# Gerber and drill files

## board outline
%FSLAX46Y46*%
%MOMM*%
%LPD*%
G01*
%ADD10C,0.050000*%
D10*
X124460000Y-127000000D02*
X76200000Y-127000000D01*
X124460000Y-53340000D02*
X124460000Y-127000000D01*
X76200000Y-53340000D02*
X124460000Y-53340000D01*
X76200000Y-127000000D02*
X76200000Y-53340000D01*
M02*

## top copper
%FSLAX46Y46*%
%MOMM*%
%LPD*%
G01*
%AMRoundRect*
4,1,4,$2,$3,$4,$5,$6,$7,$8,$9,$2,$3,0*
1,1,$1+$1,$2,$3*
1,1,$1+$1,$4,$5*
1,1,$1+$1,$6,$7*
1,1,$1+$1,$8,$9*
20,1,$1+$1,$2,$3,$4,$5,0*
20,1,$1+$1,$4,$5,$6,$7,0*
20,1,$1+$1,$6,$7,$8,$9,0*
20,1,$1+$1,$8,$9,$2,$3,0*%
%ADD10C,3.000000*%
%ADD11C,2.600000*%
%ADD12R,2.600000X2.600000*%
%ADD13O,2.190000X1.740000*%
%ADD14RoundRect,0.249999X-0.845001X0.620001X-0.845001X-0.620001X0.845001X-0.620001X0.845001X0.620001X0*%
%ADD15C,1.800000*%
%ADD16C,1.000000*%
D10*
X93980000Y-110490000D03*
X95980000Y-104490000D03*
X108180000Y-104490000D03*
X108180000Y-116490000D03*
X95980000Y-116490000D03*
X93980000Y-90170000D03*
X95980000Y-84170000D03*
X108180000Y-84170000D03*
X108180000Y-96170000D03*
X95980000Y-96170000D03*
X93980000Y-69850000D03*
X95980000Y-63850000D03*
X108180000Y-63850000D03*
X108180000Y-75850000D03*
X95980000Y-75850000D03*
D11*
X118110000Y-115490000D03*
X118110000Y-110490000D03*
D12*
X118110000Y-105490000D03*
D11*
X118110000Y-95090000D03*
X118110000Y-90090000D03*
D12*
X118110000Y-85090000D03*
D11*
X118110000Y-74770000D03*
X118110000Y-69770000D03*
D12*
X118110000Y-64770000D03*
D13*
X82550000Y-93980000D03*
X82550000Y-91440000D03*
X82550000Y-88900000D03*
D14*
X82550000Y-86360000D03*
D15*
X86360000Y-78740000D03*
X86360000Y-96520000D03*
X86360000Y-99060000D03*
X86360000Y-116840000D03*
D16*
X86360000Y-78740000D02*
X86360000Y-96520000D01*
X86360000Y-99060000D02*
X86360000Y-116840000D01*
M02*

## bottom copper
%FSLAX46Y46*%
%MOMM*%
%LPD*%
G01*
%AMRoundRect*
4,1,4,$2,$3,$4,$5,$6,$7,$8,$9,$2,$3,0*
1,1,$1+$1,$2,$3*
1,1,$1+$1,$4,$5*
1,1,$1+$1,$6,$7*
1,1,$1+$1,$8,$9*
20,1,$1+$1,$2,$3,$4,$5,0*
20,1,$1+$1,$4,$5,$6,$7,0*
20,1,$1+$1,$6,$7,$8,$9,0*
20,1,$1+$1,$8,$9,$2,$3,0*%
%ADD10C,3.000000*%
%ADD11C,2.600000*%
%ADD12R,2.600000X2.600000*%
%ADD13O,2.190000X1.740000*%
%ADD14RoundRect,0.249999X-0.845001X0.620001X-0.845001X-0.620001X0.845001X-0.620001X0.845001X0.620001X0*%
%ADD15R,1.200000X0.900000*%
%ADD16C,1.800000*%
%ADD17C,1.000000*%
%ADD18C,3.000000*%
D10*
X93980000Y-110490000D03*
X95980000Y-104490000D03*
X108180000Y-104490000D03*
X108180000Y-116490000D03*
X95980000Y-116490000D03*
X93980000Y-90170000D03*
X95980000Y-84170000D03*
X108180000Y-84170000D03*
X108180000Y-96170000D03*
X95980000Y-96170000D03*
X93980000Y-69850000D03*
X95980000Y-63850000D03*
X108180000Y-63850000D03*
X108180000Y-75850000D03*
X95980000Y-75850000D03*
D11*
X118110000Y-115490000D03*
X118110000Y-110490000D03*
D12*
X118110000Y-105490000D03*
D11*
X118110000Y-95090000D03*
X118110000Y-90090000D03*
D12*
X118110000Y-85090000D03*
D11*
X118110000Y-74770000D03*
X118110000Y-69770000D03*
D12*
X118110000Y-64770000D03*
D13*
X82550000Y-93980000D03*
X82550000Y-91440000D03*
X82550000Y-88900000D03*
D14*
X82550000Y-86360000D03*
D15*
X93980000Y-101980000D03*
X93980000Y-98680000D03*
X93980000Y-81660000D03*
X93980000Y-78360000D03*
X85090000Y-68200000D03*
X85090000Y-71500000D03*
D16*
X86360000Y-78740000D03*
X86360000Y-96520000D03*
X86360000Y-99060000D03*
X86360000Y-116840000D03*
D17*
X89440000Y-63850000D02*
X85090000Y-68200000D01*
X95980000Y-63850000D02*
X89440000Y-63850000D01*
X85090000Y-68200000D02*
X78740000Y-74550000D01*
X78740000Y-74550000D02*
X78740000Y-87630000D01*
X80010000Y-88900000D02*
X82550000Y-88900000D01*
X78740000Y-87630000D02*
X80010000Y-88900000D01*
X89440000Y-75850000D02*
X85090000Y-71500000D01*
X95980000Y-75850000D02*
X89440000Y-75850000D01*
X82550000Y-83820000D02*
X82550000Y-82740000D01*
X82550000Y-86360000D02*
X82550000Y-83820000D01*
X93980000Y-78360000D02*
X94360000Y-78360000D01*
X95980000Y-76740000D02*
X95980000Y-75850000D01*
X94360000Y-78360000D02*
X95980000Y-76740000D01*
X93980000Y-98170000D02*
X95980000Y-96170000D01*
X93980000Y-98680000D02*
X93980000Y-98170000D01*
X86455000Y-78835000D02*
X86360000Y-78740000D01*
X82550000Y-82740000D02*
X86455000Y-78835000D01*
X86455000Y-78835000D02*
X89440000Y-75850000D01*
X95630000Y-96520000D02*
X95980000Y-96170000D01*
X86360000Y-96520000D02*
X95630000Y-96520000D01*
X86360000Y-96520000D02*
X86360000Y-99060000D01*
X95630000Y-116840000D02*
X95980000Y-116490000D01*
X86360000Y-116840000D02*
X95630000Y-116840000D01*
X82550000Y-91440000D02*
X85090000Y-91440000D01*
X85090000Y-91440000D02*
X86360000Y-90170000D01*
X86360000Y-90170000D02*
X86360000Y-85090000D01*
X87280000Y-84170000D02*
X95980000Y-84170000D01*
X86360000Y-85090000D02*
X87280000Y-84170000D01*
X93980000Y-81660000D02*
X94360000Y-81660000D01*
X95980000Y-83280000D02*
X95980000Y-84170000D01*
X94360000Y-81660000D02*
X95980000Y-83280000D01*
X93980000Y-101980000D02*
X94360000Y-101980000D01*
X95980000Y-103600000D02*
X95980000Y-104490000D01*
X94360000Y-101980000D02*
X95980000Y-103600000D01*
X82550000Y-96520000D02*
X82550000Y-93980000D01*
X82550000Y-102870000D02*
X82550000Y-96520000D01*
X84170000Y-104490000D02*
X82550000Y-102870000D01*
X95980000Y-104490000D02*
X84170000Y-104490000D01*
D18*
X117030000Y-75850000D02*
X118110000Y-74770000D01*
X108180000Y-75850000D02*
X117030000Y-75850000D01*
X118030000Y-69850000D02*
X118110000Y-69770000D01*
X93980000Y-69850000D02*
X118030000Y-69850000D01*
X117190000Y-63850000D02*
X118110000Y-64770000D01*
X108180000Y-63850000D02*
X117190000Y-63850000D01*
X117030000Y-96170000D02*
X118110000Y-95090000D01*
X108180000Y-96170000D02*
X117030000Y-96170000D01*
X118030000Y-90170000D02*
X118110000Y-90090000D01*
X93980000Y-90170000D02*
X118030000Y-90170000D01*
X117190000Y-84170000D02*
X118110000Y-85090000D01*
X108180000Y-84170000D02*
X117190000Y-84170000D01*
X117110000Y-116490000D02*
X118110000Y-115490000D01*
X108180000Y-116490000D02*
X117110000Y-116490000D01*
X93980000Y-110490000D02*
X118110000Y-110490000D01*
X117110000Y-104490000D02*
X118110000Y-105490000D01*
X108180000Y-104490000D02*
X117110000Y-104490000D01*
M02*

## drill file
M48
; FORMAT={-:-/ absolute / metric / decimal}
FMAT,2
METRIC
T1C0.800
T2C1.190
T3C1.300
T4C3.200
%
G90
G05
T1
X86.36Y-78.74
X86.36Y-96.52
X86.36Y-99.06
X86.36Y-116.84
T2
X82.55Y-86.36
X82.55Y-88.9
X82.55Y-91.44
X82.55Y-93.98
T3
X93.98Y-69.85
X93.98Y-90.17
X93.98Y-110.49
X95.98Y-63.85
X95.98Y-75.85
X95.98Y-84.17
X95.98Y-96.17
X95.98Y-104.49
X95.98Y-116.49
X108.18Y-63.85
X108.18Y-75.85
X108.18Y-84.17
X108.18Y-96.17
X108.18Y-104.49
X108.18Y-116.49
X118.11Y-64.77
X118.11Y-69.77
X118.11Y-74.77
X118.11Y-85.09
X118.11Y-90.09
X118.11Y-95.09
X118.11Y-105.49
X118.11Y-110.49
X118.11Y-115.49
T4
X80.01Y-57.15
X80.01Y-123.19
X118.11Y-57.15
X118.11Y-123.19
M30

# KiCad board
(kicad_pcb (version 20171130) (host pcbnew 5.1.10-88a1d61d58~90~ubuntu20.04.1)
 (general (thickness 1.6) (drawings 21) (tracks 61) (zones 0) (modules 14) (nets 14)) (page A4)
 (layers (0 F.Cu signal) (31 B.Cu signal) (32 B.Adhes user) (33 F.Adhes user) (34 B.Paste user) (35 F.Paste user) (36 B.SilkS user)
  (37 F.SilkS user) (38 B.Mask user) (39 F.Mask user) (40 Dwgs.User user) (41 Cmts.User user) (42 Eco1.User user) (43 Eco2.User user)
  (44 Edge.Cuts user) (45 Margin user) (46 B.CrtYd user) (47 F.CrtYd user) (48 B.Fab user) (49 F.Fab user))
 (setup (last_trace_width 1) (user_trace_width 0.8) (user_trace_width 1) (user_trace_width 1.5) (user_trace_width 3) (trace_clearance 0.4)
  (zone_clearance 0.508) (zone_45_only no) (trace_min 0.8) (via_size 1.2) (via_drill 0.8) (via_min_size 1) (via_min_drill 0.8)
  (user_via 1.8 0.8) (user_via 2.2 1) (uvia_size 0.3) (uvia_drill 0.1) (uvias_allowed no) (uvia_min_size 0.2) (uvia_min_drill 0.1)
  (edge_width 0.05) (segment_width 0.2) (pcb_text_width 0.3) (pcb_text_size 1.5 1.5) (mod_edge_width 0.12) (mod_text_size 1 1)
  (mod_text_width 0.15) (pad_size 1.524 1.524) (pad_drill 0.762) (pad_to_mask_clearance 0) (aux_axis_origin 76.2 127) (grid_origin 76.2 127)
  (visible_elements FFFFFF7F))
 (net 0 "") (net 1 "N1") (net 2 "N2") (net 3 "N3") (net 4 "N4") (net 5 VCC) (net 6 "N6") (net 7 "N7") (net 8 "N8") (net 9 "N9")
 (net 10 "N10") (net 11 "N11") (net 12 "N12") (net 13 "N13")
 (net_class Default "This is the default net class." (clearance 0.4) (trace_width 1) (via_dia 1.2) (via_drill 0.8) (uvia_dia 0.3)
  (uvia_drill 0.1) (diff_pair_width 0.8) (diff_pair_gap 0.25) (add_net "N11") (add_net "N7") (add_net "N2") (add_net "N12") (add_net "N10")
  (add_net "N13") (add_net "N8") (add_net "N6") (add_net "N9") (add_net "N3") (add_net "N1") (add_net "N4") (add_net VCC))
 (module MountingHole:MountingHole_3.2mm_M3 (layer F.Cu) (at 118.11 123.19)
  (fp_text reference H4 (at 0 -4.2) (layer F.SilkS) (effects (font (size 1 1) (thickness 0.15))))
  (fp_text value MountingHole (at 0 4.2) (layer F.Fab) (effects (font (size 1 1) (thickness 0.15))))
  (pad 1 np_thru_hole circle (at 0 0) (size 3.2 3.2) (drill 3.2) (layers *.Cu *.Mask)))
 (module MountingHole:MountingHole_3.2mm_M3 (layer F.Cu) (at 118.11 57.15)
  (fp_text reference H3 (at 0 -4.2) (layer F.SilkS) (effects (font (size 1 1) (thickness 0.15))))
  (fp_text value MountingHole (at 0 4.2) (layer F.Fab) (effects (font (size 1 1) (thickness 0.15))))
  (pad 1 np_thru_hole circle (at 0 0) (size 3.2 3.2) (drill 3.2) (layers *.Cu *.Mask)))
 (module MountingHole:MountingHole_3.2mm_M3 (layer F.Cu) (at 80.01 123.19)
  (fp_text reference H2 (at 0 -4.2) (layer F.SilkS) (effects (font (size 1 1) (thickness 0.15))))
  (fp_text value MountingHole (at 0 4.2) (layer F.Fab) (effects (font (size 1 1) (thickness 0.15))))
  (pad 1 np_thru_hole circle (at 0 0) (size 3.2 3.2) (drill 3.2) (layers *.Cu *.Mask)))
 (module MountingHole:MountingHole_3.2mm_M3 (layer F.Cu) (at 80.01 57.15)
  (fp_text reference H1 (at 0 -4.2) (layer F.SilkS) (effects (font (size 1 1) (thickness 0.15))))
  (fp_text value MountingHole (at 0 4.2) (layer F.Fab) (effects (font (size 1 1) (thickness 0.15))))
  (pad 1 np_thru_hole circle (at 0 0) (size 3.2 3.2) (drill 3.2) (layers *.Cu *.Mask)))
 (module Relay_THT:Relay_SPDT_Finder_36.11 (layer F.Cu) (at 93.98 110.49)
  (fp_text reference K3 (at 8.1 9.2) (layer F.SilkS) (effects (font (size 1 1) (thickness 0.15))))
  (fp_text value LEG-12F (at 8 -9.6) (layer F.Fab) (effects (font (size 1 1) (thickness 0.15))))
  (pad 11 thru_hole circle (at 0 0) (size 3 3) (drill 1.3) (layers *.Cu *.Mask) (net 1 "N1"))
  (pad A2 thru_hole circle (at 2 -6) (size 3 3) (drill 1.3) (layers *.Cu *.Mask) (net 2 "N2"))
  (pad 12 thru_hole circle (at 14.2 -6) (size 3 3) (drill 1.3) (layers *.Cu *.Mask) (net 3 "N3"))
  (pad 14 thru_hole circle (at 14.2 6) (size 3 3) (drill 1.3) (layers *.Cu *.Mask) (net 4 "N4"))
  (pad A1 thru_hole circle (at 2 6) (size 3 3) (drill 1.3) (layers *.Cu *.Mask) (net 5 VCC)))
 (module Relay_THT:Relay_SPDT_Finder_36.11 (layer F.Cu) (at 93.98 90.17)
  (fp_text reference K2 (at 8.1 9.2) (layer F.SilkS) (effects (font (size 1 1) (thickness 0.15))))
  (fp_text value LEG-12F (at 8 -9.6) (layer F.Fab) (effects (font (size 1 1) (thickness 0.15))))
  (pad 11 thru_hole circle (at 0 0) (size 3 3) (drill 1.3) (layers *.Cu *.Mask) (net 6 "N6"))
  (pad A2 thru_hole circle (at 2 -6) (size 3 3) (drill 1.3) (layers *.Cu *.Mask) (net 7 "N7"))
  (pad 12 thru_hole circle (at 14.2 -6) (size 3 3) (drill 1.3) (layers *.Cu *.Mask) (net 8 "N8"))
  (pad 14 thru_hole circle (at 14.2 6) (size 3 3) (drill 1.3) (layers *.Cu *.Mask) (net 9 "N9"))
  (pad A1 thru_hole circle (at 2 6) (size 3 3) (drill 1.3) (layers *.Cu *.Mask) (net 5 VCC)))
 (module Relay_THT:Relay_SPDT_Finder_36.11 (layer F.Cu) (at 93.98 69.85)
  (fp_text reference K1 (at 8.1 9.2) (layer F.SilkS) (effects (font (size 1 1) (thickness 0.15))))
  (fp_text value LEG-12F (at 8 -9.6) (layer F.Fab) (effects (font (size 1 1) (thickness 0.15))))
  (pad 11 thru_hole circle (at 0 0) (size 3 3) (drill 1.3) (layers *.Cu *.Mask) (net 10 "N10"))
  (pad A2 thru_hole circle (at 2 -6) (size 3 3) (drill 1.3) (layers *.Cu *.Mask) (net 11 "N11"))
  (pad 12 thru_hole circle (at 14.2 -6) (size 3 3) (drill 1.3) (layers *.Cu *.Mask) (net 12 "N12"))
  (pad 14 thru_hole circle (at 14.2 6) (size 3 3) (drill 1.3) (layers *.Cu *.Mask) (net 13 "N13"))
  (pad A1 thru_hole circle (at 2 6) (size 3 3) (drill 1.3) (layers *.Cu *.Mask) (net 5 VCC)))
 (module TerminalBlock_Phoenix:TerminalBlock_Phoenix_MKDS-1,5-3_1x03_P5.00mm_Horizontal (layer F.Cu) (at 118.11 105.49 270)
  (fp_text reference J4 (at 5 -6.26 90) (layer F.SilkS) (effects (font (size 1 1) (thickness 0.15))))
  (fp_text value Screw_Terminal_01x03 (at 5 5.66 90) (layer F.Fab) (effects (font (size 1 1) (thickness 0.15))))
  (pad 3 thru_hole circle (at 10 0 270) (size 2.6 2.6) (drill 1.3) (layers *.Cu *.Mask) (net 4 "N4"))
  (pad 2 thru_hole circle (at 5 0 270) (size 2.6 2.6) (drill 1.3) (layers *.Cu *.Mask) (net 1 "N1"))
  (pad 1 thru_hole rect (at 0 0 270) (size 2.6 2.6) (drill 1.3) (layers *.Cu *.Mask) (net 3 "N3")))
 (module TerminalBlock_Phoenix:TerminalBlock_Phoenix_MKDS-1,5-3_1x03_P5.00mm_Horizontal (layer F.Cu) (at 118.11 85.09 270)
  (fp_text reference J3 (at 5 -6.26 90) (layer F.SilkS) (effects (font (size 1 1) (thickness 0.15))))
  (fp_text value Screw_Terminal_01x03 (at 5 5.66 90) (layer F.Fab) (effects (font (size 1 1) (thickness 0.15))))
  (pad 3 thru_hole circle (at 10 0 270) (size 2.6 2.6) (drill 1.3) (layers *.Cu *.Mask) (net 9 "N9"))
  (pad 2 thru_hole circle (at 5 0 270) (size 2.6 2.6) (drill 1.3) (layers *.Cu *.Mask) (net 6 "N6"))
  (pad 1 thru_hole rect (at 0 0 270) (size 2.6 2.6) (drill 1.3) (layers *.Cu *.Mask) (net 8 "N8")))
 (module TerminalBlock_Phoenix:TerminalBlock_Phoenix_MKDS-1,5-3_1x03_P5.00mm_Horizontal (layer F.Cu) (at 118.11 64.77 270)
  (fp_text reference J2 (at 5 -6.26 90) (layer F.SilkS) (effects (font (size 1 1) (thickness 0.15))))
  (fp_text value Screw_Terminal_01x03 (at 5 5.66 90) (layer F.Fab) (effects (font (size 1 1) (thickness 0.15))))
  (pad 3 thru_hole circle (at 10 0 270) (size 2.6 2.6) (drill 1.3) (layers *.Cu *.Mask) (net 13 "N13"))
  (pad 2 thru_hole circle (at 5 0 270) (size 2.6 2.6) (drill 1.3) (layers *.Cu *.Mask) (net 10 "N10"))
  (pad 1 thru_hole rect (at 0 0 270) (size 2.6 2.6) (drill 1.3) (layers *.Cu *.Mask) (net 12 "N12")))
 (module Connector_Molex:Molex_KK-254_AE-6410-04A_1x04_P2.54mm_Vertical (layer F.Cu) (at 82.55 86.36 270)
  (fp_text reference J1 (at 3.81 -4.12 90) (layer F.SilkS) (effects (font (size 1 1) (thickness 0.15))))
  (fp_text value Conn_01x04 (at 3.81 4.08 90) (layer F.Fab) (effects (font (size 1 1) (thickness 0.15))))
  (pad 4 thru_hole oval (at 7.62 0 270) (size 1.74 2.19) (drill 1.19) (layers *.Cu *.Mask) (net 2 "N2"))
  (pad 3 thru_hole oval (at 5.08 0 270) (size 1.74 2.19) (drill 1.19) (layers *.Cu *.Mask) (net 7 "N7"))
  (pad 2 thru_hole oval (at 2.54 0 270) (size 1.74 2.19) (drill 1.19) (layers *.Cu *.Mask) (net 11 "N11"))
  (pad 1 thru_hole roundrect (at 0 0 270) (size 1.74 2.19) (drill 1.19) (layers *.Cu *.Mask) (roundrect_rratio 0.1436775862068966)
   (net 5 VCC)))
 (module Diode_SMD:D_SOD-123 (layer B.Cu) (at 93.98 100.33 270)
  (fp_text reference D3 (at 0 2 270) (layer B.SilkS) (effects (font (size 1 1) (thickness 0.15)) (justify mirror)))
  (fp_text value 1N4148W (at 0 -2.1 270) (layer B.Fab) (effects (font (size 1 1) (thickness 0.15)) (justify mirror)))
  (pad 2 smd rect (at 1.65 0 270) (size 0.9 1.2) (layers B.Cu B.Paste B.Mask) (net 2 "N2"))
  (pad 1 smd rect (at -1.65 0 270) (size 0.9 1.2) (layers B.Cu B.Paste B.Mask) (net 5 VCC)))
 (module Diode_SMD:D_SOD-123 (layer B.Cu) (at 93.98 80.01 270)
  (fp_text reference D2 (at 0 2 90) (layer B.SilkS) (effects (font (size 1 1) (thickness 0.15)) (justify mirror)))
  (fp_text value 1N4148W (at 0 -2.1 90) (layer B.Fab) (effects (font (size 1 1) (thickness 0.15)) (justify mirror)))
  (pad 2 smd rect (at 1.65 0 270) (size 0.9 1.2) (layers B.Cu B.Paste B.Mask) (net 7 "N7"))
  (pad 1 smd rect (at -1.65 0 270) (size 0.9 1.2) (layers B.Cu B.Paste B.Mask) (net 5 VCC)))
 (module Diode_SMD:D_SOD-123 (layer B.Cu) (at 85.09 69.85 90)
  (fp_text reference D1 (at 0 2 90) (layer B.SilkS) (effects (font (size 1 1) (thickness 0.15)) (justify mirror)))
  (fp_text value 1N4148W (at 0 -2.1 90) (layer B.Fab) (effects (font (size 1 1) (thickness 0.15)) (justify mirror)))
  (pad 2 smd rect (at 1.65 0 90) (size 0.9 1.2) (layers B.Cu B.Paste B.Mask) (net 11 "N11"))
  (pad 1 smd rect (at -1.65 0 90) (size 0.9 1.2) (layers B.Cu B.Paste B.Mask) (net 5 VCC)))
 (gr_line (start 124.46 127) (end 76.2 127) (layer Edge.Cuts) (width 0.05))
 (gr_line (start 124.46 53.34) (end 124.46 127) (layer Edge.Cuts) (width 0.05))
 (gr_line (start 76.2 53.34) (end 124.46 53.34) (layer Edge.Cuts) (width 0.05))
 (gr_line (start 76.2 127) (end 76.2 53.34) (layer Edge.Cuts) (width 0.05))
 (segment (start 89.44 63.85) (end 85.09 68.2) (width 1) (layer B.Cu) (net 11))
 (segment (start 95.98 63.85) (end 89.44 63.85) (width 1) (layer B.Cu) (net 11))
 (segment (start 85.09 68.2) (end 78.74 74.55) (width 1) (layer B.Cu) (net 11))
 (segment (start 78.74 74.55) (end 78.74 87.63) (width 1) (layer B.Cu) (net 11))
 (segment (start 80.01 88.9) (end 82.55 88.9) (width 1) (layer B.Cu) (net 11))
 (segment (start 78.74 87.63) (end 80.01 88.9) (width 1) (layer B.Cu) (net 11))
 (segment (start 89.44 75.85) (end 85.09 71.5) (width 1) (layer B.Cu) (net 5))
 (segment (start 95.98 75.85) (end 89.44 75.85) (width 1) (layer B.Cu) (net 5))
 (segment (start 82.55 83.82) (end 82.55 82.74) (width 1) (layer B.Cu) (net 5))
 (segment (start 82.55 86.36) (end 82.55 83.82) (width 1) (layer B.Cu) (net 5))
 (segment (start 93.98 78.36) (end 94.36 78.36) (width 1) (layer B.Cu) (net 5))
 (segment (start 95.98 76.74) (end 95.98 75.85) (width 1) (layer B.Cu) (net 5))
 (segment (start 94.36 78.36) (end 95.98 76.74) (width 1) (layer B.Cu) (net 5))
 (segment (start 93.98 98.17) (end 95.98 96.17) (width 1) (layer B.Cu) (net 5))
 (segment (start 93.98 98.68) (end 93.98 98.17) (width 1) (layer B.Cu) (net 5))
 (via (at 86.36 78.74) (size 1.8) (drill 0.8) (layers F.Cu B.Cu) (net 5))
 (segment (start 86.455 78.835) (end 86.36 78.74) (width 1) (layer B.Cu) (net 5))
 (segment (start 82.55 82.74) (end 86.455 78.835) (width 1) (layer B.Cu) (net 5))
 (segment (start 86.455 78.835) (end 89.44 75.85) (width 1) (layer B.Cu) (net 5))
 (via (at 86.36 96.52) (size 1.8) (drill 0.8) (layers F.Cu B.Cu) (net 5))
 (segment (start 86.36 78.74) (end 86.36 96.52) (width 1) (layer F.Cu) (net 5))
 (segment (start 95.63 96.52) (end 95.98 96.17) (width 1) (layer B.Cu) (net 5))
 (segment (start 86.36 96.52) (end 95.63 96.52) (width 1) (layer B.Cu) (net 5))
 (via (at 86.36 99.06) (size 1.8) (drill 0.8) (layers F.Cu B.Cu) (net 5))
 (segment (start 86.36 96.52) (end 86.36 99.06) (width 1) (layer B.Cu) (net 5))
 (via (at 86.36 116.84) (size 1.8) (drill 0.8) (layers F.Cu B.Cu) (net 5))
 (segment (start 86.36 99.06) (end 86.36 116.84) (width 1) (layer F.Cu) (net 5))
 (segment (start 95.63 116.84) (end 95.98 116.49) (width 1) (layer B.Cu) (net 5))
 (segment (start 86.36 116.84) (end 95.63 116.84) (width 1) (layer B.Cu) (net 5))
 (segment (start 82.55 91.44) (end 85.09 91.44) (width 1) (layer B.Cu) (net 7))
 (segment (start 85.09 91.44) (end 86.36 90.17) (width 1) (layer B.Cu) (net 7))
 (segment (start 86.36 90.17) (end 86.36 85.09) (width 1) (layer B.Cu) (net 7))
 (segment (start 87.28 84.17) (end 95.98 84.17) (width 1) (layer B.Cu) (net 7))
 (segment (start 86.36 85.09) (end 87.28 84.17) (width 1) (layer B.Cu) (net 7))
 (segment (start 93.98 81.66) (end 94.36 81.66) (width 1) (layer B.Cu) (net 7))
 (segment (start 95.98 83.28) (end 95.98 84.17) (width 1) (layer B.Cu) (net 7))
 (segment (start 94.36 81.66) (end 95.98 83.28) (width 1) (layer B.Cu) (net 7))
 (segment (start 93.98 101.98) (end 94.36 101.98) (width 1) (layer B.Cu) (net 2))
 (segment (start 95.98 103.6) (end 95.98 104.49) (width 1) (layer B.Cu) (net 2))
 (segment (start 94.36 101.98) (end 95.98 103.6) (width 1) (layer B.Cu) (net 2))
 (segment (start 82.55 96.52) (end 82.55 93.98) (width 1) (layer B.Cu) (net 2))
 (segment (start 82.55 102.87) (end 82.55 96.52) (width 1) (layer B.Cu) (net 2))
 (segment (start 84.17 104.49) (end 82.55 102.87) (width 1) (layer B.Cu) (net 2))
 (segment (start 95.98 104.49) (end 84.17 104.49) (width 1) (layer B.Cu) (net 2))
 (segment (start 117.03 75.85) (end 118.11 74.77) (width 3) (layer B.Cu) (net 13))
 (segment (start 108.18 75.85) (end 117.03 75.85) (width 3) (layer B.Cu) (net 13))
 (segment (start 118.03 69.85) (end 118.11 69.77) (width 3) (layer B.Cu) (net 10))
 (segment (start 93.98 69.85) (end 118.03 69.85) (width 3) (layer B.Cu) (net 10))
 (segment (start 117.19 63.85) (end 118.11 64.77) (width 3) (layer B.Cu) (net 12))
 (segment (start 108.18 63.85) (end 117.19 63.85) (width 3) (layer B.Cu) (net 12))
 (segment (start 117.03 96.17) (end 118.11 95.09) (width 3) (layer B.Cu) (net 9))
 (segment (start 108.18 96.17) (end 117.03 96.17) (width 3) (layer B.Cu) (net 9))
 (segment (start 118.03 90.17) (end 118.11 90.09) (width 3) (layer B.Cu) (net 6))
 (segment (start 93.98 90.17) (end 118.03 90.17) (width 3) (layer B.Cu) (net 6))
 (segment (start 117.19 84.17) (end 118.11 85.09) (width 3) (layer B.Cu) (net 8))
 (segment (start 108.18 84.17) (end 117.19 84.17) (width 3) (layer B.Cu) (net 8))
 (segment (start 117.11 116.49) (end 118.11 115.49) (width 3) (layer B.Cu) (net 4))
 (segment (start 108.18 116.49) (end 117.11 116.49) (width 3) (layer B.Cu) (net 4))
 (segment (start 93.98 110.49) (end 118.11 110.49) (width 3) (layer B.Cu) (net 1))
 (segment (start 117.11 104.49) (end 118.11 105.49) (width 3) (layer B.Cu) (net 3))
 (segment (start 108.18 104.49) (end 117.11 104.49) (width 3) (layer B.Cu) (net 3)))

